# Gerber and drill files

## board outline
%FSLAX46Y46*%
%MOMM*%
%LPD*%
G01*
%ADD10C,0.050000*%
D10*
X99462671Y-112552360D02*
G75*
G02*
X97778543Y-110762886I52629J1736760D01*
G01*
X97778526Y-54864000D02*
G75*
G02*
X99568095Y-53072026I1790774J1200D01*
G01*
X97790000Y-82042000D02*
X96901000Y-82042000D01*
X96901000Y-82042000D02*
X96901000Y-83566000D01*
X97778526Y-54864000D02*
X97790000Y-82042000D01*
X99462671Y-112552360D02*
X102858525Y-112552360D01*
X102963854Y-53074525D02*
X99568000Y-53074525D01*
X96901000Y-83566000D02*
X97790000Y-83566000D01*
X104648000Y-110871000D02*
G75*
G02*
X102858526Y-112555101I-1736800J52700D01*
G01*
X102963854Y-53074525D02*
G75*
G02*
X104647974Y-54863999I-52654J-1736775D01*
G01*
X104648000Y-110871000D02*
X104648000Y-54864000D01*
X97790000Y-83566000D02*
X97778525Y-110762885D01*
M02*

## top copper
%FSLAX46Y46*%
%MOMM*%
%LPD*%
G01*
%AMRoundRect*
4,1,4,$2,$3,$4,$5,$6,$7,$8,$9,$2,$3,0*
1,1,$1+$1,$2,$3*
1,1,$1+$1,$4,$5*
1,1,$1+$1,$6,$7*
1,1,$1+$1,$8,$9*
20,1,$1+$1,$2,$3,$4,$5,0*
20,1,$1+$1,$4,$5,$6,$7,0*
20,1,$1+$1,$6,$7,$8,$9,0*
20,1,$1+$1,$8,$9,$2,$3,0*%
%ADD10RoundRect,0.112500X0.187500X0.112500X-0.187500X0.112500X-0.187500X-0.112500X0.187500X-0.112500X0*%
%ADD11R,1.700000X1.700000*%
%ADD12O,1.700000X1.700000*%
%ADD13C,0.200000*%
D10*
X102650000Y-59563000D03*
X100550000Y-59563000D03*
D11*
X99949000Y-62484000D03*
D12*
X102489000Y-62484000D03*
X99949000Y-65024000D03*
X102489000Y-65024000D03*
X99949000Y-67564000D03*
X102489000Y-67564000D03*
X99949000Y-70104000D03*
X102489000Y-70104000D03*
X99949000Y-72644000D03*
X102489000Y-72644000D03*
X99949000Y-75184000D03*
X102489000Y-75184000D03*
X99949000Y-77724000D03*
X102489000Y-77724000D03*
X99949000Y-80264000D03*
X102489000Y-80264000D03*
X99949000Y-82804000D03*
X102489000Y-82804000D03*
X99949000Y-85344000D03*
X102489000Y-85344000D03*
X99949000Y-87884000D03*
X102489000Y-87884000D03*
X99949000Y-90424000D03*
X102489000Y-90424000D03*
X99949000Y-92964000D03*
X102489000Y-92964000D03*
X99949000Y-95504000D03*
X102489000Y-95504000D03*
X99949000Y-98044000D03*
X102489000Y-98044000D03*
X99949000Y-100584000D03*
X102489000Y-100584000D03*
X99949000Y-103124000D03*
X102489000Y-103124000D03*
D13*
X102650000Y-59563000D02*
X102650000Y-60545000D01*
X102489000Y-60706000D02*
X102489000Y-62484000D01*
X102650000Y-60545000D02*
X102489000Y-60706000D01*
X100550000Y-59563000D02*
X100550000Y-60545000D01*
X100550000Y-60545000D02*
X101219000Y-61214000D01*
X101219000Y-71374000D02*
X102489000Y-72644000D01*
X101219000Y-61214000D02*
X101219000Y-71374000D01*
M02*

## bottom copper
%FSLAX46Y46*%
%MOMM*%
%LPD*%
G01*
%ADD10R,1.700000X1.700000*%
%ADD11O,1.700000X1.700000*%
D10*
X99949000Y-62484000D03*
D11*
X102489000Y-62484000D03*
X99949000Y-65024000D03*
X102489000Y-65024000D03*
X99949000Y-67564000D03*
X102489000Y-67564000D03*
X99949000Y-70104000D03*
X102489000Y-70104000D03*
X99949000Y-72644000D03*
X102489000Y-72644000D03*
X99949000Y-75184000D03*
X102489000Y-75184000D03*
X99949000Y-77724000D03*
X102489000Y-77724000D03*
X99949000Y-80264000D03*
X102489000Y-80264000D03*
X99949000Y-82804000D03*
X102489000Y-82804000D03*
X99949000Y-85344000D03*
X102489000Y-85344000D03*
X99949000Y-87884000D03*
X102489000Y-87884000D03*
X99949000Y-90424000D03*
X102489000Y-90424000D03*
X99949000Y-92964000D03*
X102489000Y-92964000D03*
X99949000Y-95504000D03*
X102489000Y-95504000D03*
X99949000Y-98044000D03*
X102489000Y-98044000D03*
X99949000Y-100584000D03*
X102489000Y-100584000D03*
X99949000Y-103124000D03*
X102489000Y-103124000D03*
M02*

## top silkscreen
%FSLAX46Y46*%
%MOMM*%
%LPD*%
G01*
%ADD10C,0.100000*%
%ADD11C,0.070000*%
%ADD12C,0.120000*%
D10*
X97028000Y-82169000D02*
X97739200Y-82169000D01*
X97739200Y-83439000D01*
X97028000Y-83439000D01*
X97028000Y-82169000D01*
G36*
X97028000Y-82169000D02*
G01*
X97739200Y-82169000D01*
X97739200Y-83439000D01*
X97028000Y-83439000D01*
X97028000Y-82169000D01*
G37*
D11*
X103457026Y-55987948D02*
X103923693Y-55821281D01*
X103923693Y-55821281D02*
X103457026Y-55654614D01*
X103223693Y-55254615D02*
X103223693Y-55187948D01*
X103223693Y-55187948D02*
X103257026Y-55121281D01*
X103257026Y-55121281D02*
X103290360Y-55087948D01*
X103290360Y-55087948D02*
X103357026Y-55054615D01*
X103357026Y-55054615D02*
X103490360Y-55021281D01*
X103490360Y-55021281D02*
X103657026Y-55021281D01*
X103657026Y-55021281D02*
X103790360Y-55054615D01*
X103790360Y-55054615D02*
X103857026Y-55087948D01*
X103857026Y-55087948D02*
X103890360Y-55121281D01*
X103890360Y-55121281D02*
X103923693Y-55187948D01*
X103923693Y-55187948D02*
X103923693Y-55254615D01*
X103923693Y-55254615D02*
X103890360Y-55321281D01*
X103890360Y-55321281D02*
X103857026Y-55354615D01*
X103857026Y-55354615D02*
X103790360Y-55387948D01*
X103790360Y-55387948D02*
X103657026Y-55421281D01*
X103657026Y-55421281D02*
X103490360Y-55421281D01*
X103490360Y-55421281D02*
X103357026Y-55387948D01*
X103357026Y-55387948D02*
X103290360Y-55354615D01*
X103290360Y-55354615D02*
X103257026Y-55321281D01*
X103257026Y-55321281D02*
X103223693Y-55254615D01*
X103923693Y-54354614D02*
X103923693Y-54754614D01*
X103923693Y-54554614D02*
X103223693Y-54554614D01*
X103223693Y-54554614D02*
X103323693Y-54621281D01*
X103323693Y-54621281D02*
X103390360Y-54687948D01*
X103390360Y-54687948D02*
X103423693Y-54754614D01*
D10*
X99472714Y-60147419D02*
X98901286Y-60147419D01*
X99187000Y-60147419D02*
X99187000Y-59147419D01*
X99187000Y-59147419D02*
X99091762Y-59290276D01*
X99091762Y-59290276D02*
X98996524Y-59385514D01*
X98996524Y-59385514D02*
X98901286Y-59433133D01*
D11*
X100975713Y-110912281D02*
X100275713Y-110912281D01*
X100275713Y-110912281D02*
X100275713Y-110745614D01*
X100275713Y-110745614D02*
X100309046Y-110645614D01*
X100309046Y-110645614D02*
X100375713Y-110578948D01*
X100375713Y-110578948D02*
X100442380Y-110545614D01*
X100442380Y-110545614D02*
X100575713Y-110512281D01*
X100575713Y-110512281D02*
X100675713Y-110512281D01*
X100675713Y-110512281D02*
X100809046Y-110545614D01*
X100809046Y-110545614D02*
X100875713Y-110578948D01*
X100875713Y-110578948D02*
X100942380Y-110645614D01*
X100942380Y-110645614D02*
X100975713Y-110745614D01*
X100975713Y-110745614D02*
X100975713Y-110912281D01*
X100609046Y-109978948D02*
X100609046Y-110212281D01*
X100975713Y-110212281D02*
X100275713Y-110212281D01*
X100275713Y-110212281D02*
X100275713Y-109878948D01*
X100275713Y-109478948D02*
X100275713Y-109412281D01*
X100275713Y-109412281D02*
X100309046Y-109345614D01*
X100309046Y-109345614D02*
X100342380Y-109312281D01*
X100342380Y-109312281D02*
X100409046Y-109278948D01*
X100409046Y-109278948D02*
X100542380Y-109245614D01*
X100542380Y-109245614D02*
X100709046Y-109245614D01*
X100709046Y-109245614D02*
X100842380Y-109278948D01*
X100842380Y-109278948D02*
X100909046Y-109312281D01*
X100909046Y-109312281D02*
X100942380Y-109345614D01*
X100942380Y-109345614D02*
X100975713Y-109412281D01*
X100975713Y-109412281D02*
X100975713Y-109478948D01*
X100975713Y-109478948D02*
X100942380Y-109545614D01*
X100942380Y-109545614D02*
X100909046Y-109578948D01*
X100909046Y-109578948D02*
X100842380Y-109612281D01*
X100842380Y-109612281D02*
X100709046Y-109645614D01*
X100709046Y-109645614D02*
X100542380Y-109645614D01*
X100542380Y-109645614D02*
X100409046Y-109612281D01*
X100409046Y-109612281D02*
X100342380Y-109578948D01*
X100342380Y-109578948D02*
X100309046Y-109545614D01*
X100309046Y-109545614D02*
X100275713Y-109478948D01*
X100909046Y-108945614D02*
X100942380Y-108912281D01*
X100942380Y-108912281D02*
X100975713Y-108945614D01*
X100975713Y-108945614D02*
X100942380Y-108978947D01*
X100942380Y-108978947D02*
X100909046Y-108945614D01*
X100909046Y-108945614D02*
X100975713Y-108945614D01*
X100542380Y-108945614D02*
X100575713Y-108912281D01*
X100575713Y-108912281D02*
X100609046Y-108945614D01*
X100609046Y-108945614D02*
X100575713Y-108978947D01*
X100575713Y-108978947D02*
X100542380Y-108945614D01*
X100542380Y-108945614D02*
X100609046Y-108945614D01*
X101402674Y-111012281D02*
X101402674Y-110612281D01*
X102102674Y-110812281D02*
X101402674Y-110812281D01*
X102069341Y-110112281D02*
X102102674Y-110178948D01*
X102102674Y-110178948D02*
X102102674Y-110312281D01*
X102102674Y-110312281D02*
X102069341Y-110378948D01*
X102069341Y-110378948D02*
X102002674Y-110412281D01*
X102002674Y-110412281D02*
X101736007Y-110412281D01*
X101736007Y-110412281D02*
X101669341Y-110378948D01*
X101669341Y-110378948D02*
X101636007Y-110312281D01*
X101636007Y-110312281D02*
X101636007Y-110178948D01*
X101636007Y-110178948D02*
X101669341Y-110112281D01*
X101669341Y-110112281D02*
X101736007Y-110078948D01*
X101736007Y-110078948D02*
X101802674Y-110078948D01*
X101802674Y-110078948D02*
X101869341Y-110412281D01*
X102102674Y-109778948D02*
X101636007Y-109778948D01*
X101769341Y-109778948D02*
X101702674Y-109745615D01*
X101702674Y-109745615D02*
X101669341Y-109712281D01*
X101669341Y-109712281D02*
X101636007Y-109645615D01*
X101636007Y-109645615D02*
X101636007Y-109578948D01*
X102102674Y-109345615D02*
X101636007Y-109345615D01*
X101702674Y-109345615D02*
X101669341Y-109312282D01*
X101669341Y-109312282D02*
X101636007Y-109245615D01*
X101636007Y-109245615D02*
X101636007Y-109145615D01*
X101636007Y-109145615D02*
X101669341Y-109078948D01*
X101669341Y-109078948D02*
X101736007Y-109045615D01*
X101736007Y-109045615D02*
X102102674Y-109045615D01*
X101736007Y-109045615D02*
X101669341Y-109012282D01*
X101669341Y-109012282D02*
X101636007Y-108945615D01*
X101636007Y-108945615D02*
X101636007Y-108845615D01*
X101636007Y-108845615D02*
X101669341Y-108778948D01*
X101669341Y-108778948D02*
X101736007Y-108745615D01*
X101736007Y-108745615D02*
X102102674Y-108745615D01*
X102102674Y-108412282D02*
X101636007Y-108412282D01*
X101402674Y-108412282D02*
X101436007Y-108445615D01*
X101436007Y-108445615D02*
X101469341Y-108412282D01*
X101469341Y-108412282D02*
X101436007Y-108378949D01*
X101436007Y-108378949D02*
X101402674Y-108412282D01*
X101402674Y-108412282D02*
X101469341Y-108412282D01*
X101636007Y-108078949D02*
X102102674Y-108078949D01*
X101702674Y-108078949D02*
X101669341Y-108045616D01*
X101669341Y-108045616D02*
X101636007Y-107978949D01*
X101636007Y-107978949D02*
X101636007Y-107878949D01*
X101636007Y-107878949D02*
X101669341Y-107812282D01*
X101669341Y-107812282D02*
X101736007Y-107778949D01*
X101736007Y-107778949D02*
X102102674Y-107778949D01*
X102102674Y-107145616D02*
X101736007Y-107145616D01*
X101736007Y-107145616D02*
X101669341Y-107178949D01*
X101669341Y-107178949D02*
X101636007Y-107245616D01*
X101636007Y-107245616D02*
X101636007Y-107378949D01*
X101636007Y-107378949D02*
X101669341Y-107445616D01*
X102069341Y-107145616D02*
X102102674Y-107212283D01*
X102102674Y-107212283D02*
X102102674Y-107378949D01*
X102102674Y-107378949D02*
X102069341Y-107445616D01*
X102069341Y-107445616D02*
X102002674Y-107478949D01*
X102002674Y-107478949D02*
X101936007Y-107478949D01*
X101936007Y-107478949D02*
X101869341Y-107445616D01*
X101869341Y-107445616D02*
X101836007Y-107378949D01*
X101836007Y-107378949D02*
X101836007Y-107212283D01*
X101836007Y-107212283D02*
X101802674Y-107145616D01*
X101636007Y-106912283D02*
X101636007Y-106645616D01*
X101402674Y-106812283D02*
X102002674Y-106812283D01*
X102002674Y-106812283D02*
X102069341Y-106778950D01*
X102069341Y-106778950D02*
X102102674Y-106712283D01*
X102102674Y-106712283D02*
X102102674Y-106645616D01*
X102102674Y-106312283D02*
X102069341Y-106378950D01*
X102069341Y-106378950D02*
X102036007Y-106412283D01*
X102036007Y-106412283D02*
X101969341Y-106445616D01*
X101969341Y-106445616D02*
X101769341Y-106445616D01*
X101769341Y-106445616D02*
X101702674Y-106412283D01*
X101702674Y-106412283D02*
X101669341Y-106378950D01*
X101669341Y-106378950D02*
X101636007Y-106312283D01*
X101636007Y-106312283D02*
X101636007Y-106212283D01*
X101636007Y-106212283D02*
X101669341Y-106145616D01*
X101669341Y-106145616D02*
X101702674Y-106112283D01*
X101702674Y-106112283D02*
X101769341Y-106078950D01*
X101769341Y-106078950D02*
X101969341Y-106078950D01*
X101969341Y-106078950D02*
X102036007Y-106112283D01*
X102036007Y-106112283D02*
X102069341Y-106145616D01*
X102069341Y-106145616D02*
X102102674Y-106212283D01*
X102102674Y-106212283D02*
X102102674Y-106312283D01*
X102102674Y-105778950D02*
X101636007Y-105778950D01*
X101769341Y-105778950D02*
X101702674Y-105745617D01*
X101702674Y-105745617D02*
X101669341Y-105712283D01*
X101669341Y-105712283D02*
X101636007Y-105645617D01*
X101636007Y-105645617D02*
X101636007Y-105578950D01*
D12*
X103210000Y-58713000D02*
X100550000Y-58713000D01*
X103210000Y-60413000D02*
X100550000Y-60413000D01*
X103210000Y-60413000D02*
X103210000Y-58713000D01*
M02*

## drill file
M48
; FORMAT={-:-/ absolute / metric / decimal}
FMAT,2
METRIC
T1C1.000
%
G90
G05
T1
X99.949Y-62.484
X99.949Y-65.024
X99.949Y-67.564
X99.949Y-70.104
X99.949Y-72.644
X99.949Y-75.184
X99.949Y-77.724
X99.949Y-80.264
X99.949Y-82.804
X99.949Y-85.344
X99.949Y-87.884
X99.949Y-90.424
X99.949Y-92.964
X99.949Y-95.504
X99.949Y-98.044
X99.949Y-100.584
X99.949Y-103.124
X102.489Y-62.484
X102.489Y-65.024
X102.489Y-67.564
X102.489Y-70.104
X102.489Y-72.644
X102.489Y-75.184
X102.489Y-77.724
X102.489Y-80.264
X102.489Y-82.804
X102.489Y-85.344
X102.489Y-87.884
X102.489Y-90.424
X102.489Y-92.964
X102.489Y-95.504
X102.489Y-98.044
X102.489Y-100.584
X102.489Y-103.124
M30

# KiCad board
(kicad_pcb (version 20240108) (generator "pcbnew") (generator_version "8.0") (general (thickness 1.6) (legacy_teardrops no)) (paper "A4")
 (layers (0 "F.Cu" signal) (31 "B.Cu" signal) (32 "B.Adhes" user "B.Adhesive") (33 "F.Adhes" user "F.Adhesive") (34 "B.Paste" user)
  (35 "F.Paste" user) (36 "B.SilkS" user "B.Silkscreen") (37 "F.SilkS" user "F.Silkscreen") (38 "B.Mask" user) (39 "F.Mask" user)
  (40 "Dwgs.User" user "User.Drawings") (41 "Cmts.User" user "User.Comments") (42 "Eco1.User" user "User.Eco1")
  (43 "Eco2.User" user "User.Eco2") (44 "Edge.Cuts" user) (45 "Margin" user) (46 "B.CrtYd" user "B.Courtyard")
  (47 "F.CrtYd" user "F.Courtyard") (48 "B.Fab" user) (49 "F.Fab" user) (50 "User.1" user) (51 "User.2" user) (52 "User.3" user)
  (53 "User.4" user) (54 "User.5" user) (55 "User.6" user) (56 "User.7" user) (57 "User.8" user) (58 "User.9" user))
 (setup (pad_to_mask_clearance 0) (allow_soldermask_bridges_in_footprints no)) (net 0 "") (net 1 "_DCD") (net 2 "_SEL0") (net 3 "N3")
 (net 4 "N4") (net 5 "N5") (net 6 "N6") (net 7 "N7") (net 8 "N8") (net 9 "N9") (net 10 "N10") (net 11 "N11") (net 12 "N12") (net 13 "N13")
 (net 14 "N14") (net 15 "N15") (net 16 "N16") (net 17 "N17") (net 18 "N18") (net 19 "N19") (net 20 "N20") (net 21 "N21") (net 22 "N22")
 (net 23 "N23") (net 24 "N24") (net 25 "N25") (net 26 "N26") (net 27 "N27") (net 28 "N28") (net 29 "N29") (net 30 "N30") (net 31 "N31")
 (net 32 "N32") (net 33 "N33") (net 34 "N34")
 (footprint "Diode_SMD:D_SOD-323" (layer "F.Cu") (at 101.6 59.563 180)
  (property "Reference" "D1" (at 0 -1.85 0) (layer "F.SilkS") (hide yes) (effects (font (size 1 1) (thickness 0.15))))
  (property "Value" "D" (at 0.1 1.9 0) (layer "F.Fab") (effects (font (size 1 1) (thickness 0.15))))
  (fp_line (start -1.61 0.85) (end 1.05 0.85) (stroke (width 0.12) (type solid)) (layer "F.SilkS"))
  (fp_line (start -1.61 -0.85) (end 1.05 -0.85) (stroke (width 0.12) (type solid)) (layer "F.SilkS"))
  (fp_line (start -1.61 -0.85) (end -1.61 0.85) (stroke (width 0.12) (type solid)) (layer "F.SilkS"))
  (pad "1" smd roundrect (at -1.05 0 180) (size 0.6 0.45) (layers "F.Cu" "F.Paste" "F.Mask") (roundrect_rratio 0.25) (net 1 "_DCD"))
  (pad "2" smd roundrect (at 1.05 0 180) (size 0.6 0.45) (layers "F.Cu" "F.Paste" "F.Mask") (roundrect_rratio 0.25) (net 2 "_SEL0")))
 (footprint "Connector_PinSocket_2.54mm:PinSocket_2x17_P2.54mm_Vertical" (layer "B.Cu") (at 99.949 62.484 180)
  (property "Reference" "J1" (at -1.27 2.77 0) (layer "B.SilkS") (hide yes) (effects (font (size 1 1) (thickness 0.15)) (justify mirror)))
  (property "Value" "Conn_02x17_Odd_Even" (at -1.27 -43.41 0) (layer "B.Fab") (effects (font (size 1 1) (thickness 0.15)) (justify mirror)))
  (pad "1" thru_hole rect (at 0 0 180) (size 1.7 1.7) (drill 1) (layers "*.Cu" "*.Mask") (remove_unused_layers no) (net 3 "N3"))
  (pad "2" thru_hole oval (at -2.54 0 180) (size 1.7 1.7) (drill 1) (layers "*.Cu" "*.Mask") (remove_unused_layers no) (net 1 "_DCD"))
  (pad "3" thru_hole oval (at 0 -2.54 180) (size 1.7 1.7) (drill 1) (layers "*.Cu" "*.Mask") (remove_unused_layers no) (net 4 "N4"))
  (pad "4" thru_hole oval (at -2.54 -2.54 180) (size 1.7 1.7) (drill 1) (layers "*.Cu" "*.Mask") (remove_unused_layers no) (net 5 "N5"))
  (pad "5" thru_hole oval (at 0 -5.08 180) (size 1.7 1.7) (drill 1) (layers "*.Cu" "*.Mask") (remove_unused_layers no) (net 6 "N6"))
  (pad "6" thru_hole oval (at -2.54 -5.08 180) (size 1.7 1.7) (drill 1) (layers "*.Cu" "*.Mask") (remove_unused_layers no) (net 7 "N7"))
  (pad "7" thru_hole oval (at 0 -7.62 180) (size 1.7 1.7) (drill 1) (layers "*.Cu" "*.Mask") (remove_unused_layers no) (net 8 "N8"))
  (pad "8" thru_hole oval (at -2.54 -7.62 180) (size 1.7 1.7) (drill 1) (layers "*.Cu" "*.Mask") (remove_unused_layers no) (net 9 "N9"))
  (pad "9" thru_hole oval (at 0 -10.16 180) (size 1.7 1.7) (drill 1) (layers "*.Cu" "*.Mask") (remove_unused_layers no) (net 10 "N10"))
  (pad "10" thru_hole oval (at -2.54 -10.16 180) (size 1.7 1.7) (drill 1) (layers "*.Cu" "*.Mask") (remove_unused_layers no) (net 2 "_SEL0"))
  (pad "11" thru_hole oval (at 0 -12.7 180) (size 1.7 1.7) (drill 1) (layers "*.Cu" "*.Mask") (remove_unused_layers no) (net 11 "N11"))
  (pad "12" thru_hole oval (at -2.54 -12.7 180) (size 1.7 1.7) (drill 1) (layers "*.Cu" "*.Mask") (remove_unused_layers no) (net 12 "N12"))
  (pad "13" thru_hole oval (at 0 -15.24 180) (size 1.7 1.7) (drill 1) (layers "*.Cu" "*.Mask") (remove_unused_layers no) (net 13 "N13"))
  (pad "14" thru_hole oval (at -2.54 -15.24 180) (size 1.7 1.7) (drill 1) (layers "*.Cu" "*.Mask") (remove_unused_layers no) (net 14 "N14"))
  (pad "15" thru_hole oval (at 0 -17.78 180) (size 1.7 1.7) (drill 1) (layers "*.Cu" "*.Mask") (remove_unused_layers no) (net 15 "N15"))
  (pad "16" thru_hole oval (at -2.54 -17.78 180) (size 1.7 1.7) (drill 1) (layers "*.Cu" "*.Mask") (remove_unused_layers no) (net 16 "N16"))
  (pad "17" thru_hole oval (at 0 -20.32 180) (size 1.7 1.7) (drill 1) (layers "*.Cu" "*.Mask") (remove_unused_layers no) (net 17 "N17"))
  (pad "18" thru_hole oval (at -2.54 -20.32 180) (size 1.7 1.7) (drill 1) (layers "*.Cu" "*.Mask") (remove_unused_layers no) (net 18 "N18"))
  (pad "19" thru_hole oval (at 0 -22.86 180) (size 1.7 1.7) (drill 1) (layers "*.Cu" "*.Mask") (remove_unused_layers no) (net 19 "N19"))
  (pad "20" thru_hole oval (at -2.54 -22.86 180) (size 1.7 1.7) (drill 1) (layers "*.Cu" "*.Mask") (remove_unused_layers no) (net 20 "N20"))
  (pad "21" thru_hole oval (at 0 -25.4 180) (size 1.7 1.7) (drill 1) (layers "*.Cu" "*.Mask") (remove_unused_layers no) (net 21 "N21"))
  (pad "22" thru_hole oval (at -2.54 -25.4 180) (size 1.7 1.7) (drill 1) (layers "*.Cu" "*.Mask") (remove_unused_layers no) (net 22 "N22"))
  (pad "23" thru_hole oval (at 0 -27.94 180) (size 1.7 1.7) (drill 1) (layers "*.Cu" "*.Mask") (remove_unused_layers no) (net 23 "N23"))
  (pad "24" thru_hole oval (at -2.54 -27.94 180) (size 1.7 1.7) (drill 1) (layers "*.Cu" "*.Mask") (remove_unused_layers no) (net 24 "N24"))
  (pad "25" thru_hole oval (at 0 -30.48 180) (size 1.7 1.7) (drill 1) (layers "*.Cu" "*.Mask") (remove_unused_layers no) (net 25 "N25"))
  (pad "26" thru_hole oval (at -2.54 -30.48 180) (size 1.7 1.7) (drill 1) (layers "*.Cu" "*.Mask") (remove_unused_layers no) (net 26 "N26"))
  (pad "27" thru_hole oval (at 0 -33.02 180) (size 1.7 1.7) (drill 1) (layers "*.Cu" "*.Mask") (remove_unused_layers no) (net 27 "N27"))
  (pad "28" thru_hole oval (at -2.54 -33.02 180) (size 1.7 1.7) (drill 1) (layers "*.Cu" "*.Mask") (remove_unused_layers no) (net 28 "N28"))
  (pad "29" thru_hole oval (at 0 -35.56 180) (size 1.7 1.7) (drill 1) (layers "*.Cu" "*.Mask") (remove_unused_layers no) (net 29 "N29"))
  (pad "30" thru_hole oval (at -2.54 -35.56 180) (size 1.7 1.7) (drill 1) (layers "*.Cu" "*.Mask") (remove_unused_layers no) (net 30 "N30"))
  (pad "31" thru_hole oval (at 0 -38.1 180) (size 1.7 1.7) (drill 1) (layers "*.Cu" "*.Mask") (remove_unused_layers no) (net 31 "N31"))
  (pad "32" thru_hole oval (at -2.54 -38.1 180) (size 1.7 1.7) (drill 1) (layers "*.Cu" "*.Mask") (remove_unused_layers no) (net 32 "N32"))
  (pad "33" thru_hole oval (at 0 -40.64 180) (size 1.7 1.7) (drill 1) (layers "*.Cu" "*.Mask") (remove_unused_layers no) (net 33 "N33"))
  (pad "34" thru_hole oval (at -2.54 -40.64 180) (size 1.7 1.7) (drill 1) (layers "*.Cu" "*.Mask") (remove_unused_layers no) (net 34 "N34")))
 (gr_rect (start 97.028 82.169) (end 97.7392 83.439) (stroke (width 0.1) (type solid)) (fill solid) (layer "F.SilkS"))
 (gr_arc (start 99.462671 112.55236) (mid 98.249985 112.006421) (end 97.778525 110.762885) (stroke (width 0.05) (type solid))
  (layer "Edge.Cuts"))
 (gr_arc (start 97.778526 54.864) (mid 98.302172 53.597361) (end 99.568095 53.071986) (stroke (width 0.05) (type solid)) (layer "Edge.Cuts"))
 (gr_line (start 97.79 82.042) (end 96.901 82.042) (stroke (width 0.05) (type default)) (layer "Edge.Cuts"))
 (gr_line (start 96.901 82.042) (end 96.901 83.566) (stroke (width 0.05) (type default)) (layer "Edge.Cuts"))
 (gr_line (start 97.778526 54.864) (end 97.79 82.042) (stroke (width 0.05) (type default)) (layer "Edge.Cuts"))
 (gr_line (start 99.462671 112.55236) (end 102.858525 112.55236) (stroke (width 0.05) (type default)) (layer "Edge.Cuts"))
 (gr_line (start 102.963854 53.074525) (end 99.568 53.074525) (stroke (width 0.05) (type default)) (layer "Edge.Cuts"))
 (gr_line (start 96.901 83.566) (end 97.79 83.566) (stroke (width 0.05) (type default)) (layer "Edge.Cuts"))
 (gr_arc (start 104.648 110.871) (mid 104.102061 112.083686) (end 102.858525 112.555146) (stroke (width 0.05) (type solid))
  (layer "Edge.Cuts"))
 (gr_arc (start 102.963854 53.074525) (mid 104.17654 53.620464) (end 104.648 54.864) (stroke (width 0.05) (type solid)) (layer "Edge.Cuts"))
 (gr_line (start 104.648 110.871) (end 104.648 54.864) (stroke (width 0.05) (type default)) (layer "Edge.Cuts"))
 (gr_line (start 97.79 83.566) (end 97.778525 110.762885) (stroke (width 0.05) (type default)) (layer "Edge.Cuts"))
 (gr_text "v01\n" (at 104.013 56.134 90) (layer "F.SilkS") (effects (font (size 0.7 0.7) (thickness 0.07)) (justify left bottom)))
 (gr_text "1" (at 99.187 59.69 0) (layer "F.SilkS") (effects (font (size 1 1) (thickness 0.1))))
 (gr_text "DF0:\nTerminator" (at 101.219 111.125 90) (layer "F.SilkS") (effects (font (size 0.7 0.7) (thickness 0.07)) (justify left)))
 (segment (start 102.65 59.563) (end 102.65 60.545) (width 0.2) (layer "F.Cu") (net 1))
 (segment (start 102.489 60.706) (end 102.489 62.484) (width 0.2) (layer "F.Cu") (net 1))
 (segment (start 102.65 60.545) (end 102.489 60.706) (width 0.2) (layer "F.Cu") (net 1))
 (segment (start 100.55 59.563) (end 100.55 60.545) (width 0.2) (layer "F.Cu") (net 2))
 (segment (start 100.55 60.545) (end 101.219 61.214) (width 0.2) (layer "F.Cu") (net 2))
 (segment (start 101.219 71.374) (end 102.489 72.644) (width 0.2) (layer "F.Cu") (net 2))
 (segment (start 101.219 61.214) (end 101.219 71.374) (width 0.2) (layer "F.Cu") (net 2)))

